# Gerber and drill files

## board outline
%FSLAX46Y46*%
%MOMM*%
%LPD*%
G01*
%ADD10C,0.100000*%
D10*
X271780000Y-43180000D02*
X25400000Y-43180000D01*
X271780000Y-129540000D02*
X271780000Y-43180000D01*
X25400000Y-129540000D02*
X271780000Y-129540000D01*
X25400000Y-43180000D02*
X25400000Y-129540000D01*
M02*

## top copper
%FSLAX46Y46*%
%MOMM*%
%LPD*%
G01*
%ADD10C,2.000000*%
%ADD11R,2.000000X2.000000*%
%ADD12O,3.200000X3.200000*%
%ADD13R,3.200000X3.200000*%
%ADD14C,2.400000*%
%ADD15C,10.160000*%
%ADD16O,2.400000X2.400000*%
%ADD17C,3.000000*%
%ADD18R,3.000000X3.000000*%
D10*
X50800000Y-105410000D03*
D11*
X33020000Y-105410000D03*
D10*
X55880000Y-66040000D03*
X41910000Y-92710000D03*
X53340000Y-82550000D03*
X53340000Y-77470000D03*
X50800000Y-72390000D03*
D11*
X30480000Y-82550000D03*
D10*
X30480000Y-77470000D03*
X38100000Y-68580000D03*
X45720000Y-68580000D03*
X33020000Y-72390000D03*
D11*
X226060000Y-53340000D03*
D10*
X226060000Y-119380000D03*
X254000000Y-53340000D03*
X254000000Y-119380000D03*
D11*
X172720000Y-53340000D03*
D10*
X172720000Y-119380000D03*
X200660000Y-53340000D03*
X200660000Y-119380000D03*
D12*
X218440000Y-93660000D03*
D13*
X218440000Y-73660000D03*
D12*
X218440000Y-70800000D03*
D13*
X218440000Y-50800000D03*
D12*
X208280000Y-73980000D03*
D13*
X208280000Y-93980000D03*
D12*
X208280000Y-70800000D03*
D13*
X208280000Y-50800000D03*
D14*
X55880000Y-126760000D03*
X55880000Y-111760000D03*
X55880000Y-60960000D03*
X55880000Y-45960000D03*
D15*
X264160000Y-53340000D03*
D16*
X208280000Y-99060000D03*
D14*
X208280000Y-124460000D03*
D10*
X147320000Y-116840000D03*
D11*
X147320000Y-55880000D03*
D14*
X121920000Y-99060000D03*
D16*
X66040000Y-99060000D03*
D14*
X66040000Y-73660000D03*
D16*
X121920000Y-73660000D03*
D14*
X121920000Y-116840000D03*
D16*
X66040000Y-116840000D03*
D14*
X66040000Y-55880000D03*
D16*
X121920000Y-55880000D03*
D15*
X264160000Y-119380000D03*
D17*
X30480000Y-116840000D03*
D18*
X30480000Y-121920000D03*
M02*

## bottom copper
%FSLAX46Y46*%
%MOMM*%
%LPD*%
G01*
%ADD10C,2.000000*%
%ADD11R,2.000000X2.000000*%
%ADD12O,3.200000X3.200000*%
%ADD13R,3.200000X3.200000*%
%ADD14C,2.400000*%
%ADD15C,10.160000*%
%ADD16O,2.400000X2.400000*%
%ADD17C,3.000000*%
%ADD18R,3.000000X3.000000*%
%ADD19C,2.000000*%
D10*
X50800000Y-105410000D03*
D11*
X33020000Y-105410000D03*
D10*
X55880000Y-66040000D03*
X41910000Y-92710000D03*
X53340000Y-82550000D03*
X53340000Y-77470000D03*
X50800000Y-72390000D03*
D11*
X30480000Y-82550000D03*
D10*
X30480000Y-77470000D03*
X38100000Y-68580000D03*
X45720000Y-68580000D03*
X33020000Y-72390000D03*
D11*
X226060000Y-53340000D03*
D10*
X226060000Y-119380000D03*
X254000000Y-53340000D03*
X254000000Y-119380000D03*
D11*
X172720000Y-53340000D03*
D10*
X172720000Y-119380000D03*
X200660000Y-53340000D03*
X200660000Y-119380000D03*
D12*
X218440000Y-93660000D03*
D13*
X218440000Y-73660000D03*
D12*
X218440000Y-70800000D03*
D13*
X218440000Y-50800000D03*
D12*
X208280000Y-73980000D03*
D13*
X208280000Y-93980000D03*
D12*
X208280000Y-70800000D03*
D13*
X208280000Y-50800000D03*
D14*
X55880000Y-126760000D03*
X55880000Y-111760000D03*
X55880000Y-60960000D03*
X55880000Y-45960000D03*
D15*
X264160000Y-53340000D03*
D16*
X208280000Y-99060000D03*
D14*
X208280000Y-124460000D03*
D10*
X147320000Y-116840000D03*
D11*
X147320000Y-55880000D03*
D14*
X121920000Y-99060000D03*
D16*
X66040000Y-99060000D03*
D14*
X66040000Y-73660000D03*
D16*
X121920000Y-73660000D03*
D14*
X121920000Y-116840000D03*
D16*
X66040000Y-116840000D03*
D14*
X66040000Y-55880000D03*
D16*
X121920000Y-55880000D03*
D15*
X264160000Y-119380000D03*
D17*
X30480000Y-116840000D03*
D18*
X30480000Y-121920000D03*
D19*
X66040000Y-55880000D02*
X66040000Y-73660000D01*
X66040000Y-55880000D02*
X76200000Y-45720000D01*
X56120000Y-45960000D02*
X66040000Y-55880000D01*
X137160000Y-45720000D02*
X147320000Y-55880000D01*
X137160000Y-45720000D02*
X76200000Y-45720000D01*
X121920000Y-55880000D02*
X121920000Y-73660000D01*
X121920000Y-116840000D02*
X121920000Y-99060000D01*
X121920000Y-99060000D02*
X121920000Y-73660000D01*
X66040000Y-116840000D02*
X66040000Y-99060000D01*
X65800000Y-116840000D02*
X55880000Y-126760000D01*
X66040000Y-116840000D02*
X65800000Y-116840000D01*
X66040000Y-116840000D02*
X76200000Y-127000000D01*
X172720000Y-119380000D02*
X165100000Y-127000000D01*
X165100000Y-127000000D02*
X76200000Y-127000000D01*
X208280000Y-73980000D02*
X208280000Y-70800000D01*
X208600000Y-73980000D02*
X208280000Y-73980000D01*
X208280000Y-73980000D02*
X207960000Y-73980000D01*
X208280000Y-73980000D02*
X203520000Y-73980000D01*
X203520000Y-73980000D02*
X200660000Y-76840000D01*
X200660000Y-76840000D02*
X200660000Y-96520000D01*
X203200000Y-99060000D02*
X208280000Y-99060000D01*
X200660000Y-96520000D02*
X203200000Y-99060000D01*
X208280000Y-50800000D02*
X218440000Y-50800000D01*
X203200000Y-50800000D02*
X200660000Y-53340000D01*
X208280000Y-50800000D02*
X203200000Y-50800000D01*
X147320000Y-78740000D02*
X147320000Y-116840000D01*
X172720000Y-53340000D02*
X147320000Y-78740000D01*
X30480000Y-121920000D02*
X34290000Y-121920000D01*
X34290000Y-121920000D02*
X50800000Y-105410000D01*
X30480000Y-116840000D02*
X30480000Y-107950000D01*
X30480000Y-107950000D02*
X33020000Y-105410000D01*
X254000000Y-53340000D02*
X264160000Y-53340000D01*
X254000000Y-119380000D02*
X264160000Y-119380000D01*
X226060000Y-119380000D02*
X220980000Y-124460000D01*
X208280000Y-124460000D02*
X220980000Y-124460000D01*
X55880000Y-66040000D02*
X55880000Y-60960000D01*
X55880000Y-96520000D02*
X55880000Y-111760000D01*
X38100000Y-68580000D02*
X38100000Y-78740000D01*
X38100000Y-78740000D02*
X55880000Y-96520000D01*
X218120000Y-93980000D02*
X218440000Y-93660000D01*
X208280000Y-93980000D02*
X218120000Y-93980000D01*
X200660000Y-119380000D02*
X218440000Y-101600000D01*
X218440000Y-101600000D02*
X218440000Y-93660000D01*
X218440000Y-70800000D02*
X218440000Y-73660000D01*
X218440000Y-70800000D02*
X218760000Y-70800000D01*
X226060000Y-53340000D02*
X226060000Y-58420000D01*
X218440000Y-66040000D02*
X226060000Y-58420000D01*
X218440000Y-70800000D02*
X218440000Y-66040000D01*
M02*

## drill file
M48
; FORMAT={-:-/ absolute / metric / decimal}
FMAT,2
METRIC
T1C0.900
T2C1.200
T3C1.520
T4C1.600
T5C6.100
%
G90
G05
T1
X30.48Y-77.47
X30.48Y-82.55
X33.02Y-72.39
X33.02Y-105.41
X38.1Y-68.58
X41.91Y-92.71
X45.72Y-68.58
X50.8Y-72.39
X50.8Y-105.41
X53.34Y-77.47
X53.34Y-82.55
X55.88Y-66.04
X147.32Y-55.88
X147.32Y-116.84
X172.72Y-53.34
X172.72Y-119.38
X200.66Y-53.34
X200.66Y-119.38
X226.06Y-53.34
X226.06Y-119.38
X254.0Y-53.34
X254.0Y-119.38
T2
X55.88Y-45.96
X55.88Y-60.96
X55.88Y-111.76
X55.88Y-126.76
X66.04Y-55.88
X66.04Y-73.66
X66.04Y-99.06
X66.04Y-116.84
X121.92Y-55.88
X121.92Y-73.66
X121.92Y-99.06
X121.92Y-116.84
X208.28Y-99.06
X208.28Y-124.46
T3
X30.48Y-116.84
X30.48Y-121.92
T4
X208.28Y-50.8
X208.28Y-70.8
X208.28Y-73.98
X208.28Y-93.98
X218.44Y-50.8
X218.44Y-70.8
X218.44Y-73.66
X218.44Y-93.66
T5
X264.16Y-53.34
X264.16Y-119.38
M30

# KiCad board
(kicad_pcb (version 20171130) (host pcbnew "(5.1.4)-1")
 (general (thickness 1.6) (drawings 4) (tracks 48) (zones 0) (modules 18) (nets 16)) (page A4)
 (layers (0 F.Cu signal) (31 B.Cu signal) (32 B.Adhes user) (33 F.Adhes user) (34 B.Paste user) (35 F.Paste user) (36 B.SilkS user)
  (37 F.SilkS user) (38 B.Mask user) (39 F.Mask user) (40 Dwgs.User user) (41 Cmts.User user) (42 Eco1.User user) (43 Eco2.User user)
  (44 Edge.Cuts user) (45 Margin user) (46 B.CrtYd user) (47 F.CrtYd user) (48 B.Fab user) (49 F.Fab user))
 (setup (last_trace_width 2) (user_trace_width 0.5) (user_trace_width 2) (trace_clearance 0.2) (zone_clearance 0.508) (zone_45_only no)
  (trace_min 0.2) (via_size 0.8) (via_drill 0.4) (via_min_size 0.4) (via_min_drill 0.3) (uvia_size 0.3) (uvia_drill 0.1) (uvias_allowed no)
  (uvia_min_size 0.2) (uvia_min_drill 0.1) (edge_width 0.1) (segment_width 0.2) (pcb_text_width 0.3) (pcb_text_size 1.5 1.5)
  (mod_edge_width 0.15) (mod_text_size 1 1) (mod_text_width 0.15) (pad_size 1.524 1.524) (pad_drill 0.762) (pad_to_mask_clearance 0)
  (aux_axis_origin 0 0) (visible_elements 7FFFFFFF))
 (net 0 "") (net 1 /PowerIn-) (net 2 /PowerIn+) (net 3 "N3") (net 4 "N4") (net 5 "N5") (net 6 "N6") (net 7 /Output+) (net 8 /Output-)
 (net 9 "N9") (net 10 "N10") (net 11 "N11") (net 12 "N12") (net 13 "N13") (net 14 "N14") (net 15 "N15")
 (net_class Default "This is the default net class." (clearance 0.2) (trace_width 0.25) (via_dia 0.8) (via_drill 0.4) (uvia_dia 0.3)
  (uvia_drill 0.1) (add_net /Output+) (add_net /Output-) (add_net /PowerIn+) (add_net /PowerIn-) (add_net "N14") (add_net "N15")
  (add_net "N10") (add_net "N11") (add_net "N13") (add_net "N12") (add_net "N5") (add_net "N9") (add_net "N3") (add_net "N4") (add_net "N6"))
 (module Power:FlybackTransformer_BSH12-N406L (layer F.Cu) (at 57.15 66.04 270)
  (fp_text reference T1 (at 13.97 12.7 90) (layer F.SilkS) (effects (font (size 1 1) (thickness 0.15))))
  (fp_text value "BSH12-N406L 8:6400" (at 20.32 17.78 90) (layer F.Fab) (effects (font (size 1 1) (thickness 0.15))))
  (pad 11 thru_hole circle (at 39.37 6.35 270) (size 2 2) (drill 0.9) (layers *.Cu *.Mask) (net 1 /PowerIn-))
  (pad 10 thru_hole rect (at 39.37 24.13 270) (size 2 2) (drill 0.9) (layers *.Cu *.Mask) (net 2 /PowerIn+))
  (pad 12 thru_hole circle (at 0 1.27 270) (size 2 2) (drill 0.9) (layers *.Cu *.Mask) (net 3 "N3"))
  (pad 9 thru_hole circle (at 26.67 15.24 270) (size 2 2) (drill 0.9) (layers *.Cu *.Mask))
  (pad 8 thru_hole circle (at 16.51 3.81 270) (size 2 2) (drill 0.9) (layers *.Cu *.Mask))
  (pad 7 thru_hole circle (at 11.43 3.81 270) (size 2 2) (drill 0.9) (layers *.Cu *.Mask))
  (pad 6 thru_hole circle (at 6.35 6.35 270) (size 2 2) (drill 0.9) (layers *.Cu *.Mask))
  (pad 1 thru_hole rect (at 16.51 26.67 270) (size 2 2) (drill 0.9) (layers *.Cu *.Mask))
  (pad 2 thru_hole circle (at 11.43 26.67 270) (size 2 2) (drill 0.9) (layers *.Cu *.Mask))
  (pad 4 thru_hole circle (at 2.54 19.05 270) (size 2 2) (drill 0.9) (layers *.Cu *.Mask) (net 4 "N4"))
  (pad 5 thru_hole circle (at 2.54 11.43 270) (size 2 2) (drill 0.9) (layers *.Cu *.Mask))
  (pad 3 thru_hole circle (at 6.35 24.13 270) (size 2 2) (drill 0.9) (layers *.Cu *.Mask)))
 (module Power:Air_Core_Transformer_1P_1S (layer F.Cu) (at 226.06 53.34)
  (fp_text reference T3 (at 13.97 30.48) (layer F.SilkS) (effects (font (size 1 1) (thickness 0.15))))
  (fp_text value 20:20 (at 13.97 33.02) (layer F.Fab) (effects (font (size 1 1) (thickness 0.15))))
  (pad 1 thru_hole rect (at 0 0) (size 2 2) (drill 0.9) (layers *.Cu *.Mask) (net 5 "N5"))
  (pad 2 thru_hole circle (at 0 66.04) (size 2 2) (drill 0.9) (layers *.Cu *.Mask) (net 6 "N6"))
  (pad 4 thru_hole circle (at 27.94 0) (size 2 2) (drill 0.9) (layers *.Cu *.Mask) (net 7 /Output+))
  (pad 3 thru_hole circle (at 27.94 66.04) (size 2 2) (drill 0.9) (layers *.Cu *.Mask) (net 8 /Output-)))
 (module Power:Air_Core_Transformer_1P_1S (layer F.Cu) (at 172.72 53.34)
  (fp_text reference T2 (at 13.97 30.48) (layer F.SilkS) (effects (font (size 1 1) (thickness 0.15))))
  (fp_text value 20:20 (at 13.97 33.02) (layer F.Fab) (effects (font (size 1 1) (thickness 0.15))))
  (pad 1 thru_hole rect (at 0 0) (size 2 2) (drill 0.9) (layers *.Cu *.Mask) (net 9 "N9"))
  (pad 2 thru_hole circle (at 0 66.04) (size 2 2) (drill 0.9) (layers *.Cu *.Mask) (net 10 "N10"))
  (pad 4 thru_hole circle (at 27.94 0) (size 2 2) (drill 0.9) (layers *.Cu *.Mask) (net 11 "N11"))
  (pad 3 thru_hole circle (at 27.94 66.04) (size 2 2) (drill 0.9) (layers *.Cu *.Mask) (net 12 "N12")))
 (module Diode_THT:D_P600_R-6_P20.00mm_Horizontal (layer F.Cu) (at 218.44 73.66 270)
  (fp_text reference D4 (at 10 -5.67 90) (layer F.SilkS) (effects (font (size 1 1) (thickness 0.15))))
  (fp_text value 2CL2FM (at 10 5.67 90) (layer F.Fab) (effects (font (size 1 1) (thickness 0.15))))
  (pad 2 thru_hole oval (at 20 0 270) (size 3.2 3.2) (drill 1.6) (layers *.Cu *.Mask) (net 12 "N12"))
  (pad 1 thru_hole rect (at 0 0 270) (size 3.2 3.2) (drill 1.6) (layers *.Cu *.Mask) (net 5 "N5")))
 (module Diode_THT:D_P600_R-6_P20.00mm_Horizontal (layer F.Cu) (at 218.44 50.8 270)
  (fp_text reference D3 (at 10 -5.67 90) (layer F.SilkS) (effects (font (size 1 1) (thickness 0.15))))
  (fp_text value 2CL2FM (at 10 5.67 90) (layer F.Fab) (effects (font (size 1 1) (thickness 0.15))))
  (pad 2 thru_hole oval (at 20 0 270) (size 3.2 3.2) (drill 1.6) (layers *.Cu *.Mask) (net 5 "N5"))
  (pad 1 thru_hole rect (at 0 0 270) (size 3.2 3.2) (drill 1.6) (layers *.Cu *.Mask) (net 11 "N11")))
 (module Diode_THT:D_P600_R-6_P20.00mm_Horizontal (layer F.Cu) (at 208.28 93.98 90)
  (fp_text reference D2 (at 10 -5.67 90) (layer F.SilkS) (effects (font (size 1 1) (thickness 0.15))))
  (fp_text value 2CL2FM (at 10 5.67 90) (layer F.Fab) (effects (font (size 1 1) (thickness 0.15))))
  (pad 2 thru_hole oval (at 20 0 90) (size 3.2 3.2) (drill 1.6) (layers *.Cu *.Mask) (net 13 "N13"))
  (pad 1 thru_hole rect (at 0 0 90) (size 3.2 3.2) (drill 1.6) (layers *.Cu *.Mask) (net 12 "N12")))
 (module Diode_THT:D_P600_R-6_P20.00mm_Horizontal (layer F.Cu) (at 208.28 50.8 270)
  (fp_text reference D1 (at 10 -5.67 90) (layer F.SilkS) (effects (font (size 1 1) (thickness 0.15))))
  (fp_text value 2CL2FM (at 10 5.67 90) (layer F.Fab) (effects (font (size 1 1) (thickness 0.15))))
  (pad 2 thru_hole oval (at 20 0 270) (size 3.2 3.2) (drill 1.6) (layers *.Cu *.Mask) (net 13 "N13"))
  (pad 1 thru_hole rect (at 0 0 270) (size 3.2 3.2) (drill 1.6) (layers *.Cu *.Mask) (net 11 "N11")))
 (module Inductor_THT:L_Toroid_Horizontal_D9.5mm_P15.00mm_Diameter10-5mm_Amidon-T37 (layer F.Cu) (at 55.88 111.76 270)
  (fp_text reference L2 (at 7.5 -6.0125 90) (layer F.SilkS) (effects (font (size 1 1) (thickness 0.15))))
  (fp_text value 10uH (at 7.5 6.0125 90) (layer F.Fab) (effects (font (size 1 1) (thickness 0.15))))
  (pad 2 thru_hole circle (at 15 0 270) (size 2.4 2.4) (drill 1.2) (layers *.Cu *.Mask) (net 10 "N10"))
  (pad 1 thru_hole circle (at 0 0 270) (size 2.4 2.4) (drill 1.2) (layers *.Cu *.Mask) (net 4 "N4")))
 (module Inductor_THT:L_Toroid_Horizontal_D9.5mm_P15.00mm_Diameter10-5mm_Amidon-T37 (layer F.Cu) (at 55.88 60.96 90)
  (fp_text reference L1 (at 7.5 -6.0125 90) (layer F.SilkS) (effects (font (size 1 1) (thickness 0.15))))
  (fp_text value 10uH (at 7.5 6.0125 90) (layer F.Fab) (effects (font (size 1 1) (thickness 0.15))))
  (pad 1 thru_hole circle (at 0 0 90) (size 2.4 2.4) (drill 1.2) (layers *.Cu *.Mask) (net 3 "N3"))
  (pad 2 thru_hole circle (at 15 0 90) (size 2.4 2.4) (drill 1.2) (layers *.Cu *.Mask) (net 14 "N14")))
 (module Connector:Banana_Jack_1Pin (layer F.Cu) (at 264.16 53.34)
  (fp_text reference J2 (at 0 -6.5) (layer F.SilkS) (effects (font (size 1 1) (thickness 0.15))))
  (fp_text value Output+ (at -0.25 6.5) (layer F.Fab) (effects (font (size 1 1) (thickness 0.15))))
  (pad 1 thru_hole circle (at 0 0) (size 10.16 10.16) (drill 6.1) (layers *.Cu *.Mask) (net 7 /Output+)))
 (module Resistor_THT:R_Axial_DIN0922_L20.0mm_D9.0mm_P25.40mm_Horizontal (layer F.Cu) (at 208.28 124.46 90)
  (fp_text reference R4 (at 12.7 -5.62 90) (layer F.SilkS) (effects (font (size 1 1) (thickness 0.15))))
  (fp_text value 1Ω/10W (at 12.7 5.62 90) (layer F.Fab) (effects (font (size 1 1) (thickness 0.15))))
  (pad 2 thru_hole oval (at 25.4 0 90) (size 2.4 2.4) (drill 1.2) (layers *.Cu *.Mask) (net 13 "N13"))
  (pad 1 thru_hole circle (at 0 0 90) (size 2.4 2.4) (drill 1.2) (layers *.Cu *.Mask) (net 6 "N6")))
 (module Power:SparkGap (layer F.Cu) (at 147.32 55.88 270)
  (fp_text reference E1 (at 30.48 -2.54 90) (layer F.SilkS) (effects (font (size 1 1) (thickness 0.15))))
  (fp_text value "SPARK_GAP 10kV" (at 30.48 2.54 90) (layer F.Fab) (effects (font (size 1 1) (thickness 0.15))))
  (pad 2 thru_hole circle (at 60.96 0 270) (size 2 2) (drill 0.9) (layers *.Cu *.Mask) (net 9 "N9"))
  (pad 1 thru_hole rect (at 0 0 270) (size 2 2) (drill 0.9) (layers *.Cu *.Mask) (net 14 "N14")))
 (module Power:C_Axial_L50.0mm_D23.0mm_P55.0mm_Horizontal (layer F.Cu) (at 121.92 99.06 180)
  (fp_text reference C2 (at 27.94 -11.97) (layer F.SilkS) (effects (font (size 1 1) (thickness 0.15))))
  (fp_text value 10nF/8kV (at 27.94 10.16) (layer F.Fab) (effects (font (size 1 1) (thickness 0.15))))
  (pad 1 thru_hole circle (at 0 0 180) (size 2.4 2.4) (drill 1.2) (layers *.Cu *.Mask) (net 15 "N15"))
  (pad 2 thru_hole oval (at 55.88 0 180) (size 2.4 2.4) (drill 1.2) (layers *.Cu *.Mask) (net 10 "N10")))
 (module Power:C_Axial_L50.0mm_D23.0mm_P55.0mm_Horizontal (layer F.Cu) (at 66.04 73.66)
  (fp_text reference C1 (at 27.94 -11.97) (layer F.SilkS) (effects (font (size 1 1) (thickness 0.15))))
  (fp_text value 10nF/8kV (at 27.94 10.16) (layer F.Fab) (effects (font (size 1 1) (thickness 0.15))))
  (pad 1 thru_hole circle (at 0 0) (size 2.4 2.4) (drill 1.2) (layers *.Cu *.Mask) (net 14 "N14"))
  (pad 2 thru_hole oval (at 55.88 0) (size 2.4 2.4) (drill 1.2) (layers *.Cu *.Mask) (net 15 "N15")))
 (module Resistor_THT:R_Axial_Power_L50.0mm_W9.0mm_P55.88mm (layer F.Cu) (at 121.92 116.84 180)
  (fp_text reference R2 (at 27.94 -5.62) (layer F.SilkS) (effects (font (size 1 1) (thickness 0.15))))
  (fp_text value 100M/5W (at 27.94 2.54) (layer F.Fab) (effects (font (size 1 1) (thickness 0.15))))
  (pad 1 thru_hole circle (at 0 0 180) (size 2.4 2.4) (drill 1.2) (layers *.Cu *.Mask) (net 15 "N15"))
  (pad 2 thru_hole oval (at 55.88 0 180) (size 2.4 2.4) (drill 1.2) (layers *.Cu *.Mask) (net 10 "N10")))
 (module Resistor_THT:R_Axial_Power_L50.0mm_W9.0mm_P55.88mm (layer F.Cu) (at 66.04 55.88)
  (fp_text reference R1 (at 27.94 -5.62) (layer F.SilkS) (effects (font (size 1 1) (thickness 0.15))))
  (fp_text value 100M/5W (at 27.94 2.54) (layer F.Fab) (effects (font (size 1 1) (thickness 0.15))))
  (pad 1 thru_hole circle (at 0 0) (size 2.4 2.4) (drill 1.2) (layers *.Cu *.Mask) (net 14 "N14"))
  (pad 2 thru_hole oval (at 55.88 0) (size 2.4 2.4) (drill 1.2) (layers *.Cu *.Mask) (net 15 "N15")))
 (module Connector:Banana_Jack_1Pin (layer F.Cu) (at 264.16 119.38)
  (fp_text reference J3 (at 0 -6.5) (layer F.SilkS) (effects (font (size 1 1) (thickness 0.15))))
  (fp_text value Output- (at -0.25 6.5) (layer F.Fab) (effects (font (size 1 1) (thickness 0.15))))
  (pad 1 thru_hole circle (at 0 0) (size 10.16 10.16) (drill 6.1) (layers *.Cu *.Mask) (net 8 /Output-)))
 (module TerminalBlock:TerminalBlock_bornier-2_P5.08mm (layer F.Cu) (at 30.48 121.92 90)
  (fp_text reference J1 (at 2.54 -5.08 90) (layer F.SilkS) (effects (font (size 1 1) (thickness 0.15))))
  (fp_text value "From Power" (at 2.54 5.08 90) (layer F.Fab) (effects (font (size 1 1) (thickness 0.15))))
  (pad 2 thru_hole circle (at 5.08 0 90) (size 3 3) (drill 1.52) (layers *.Cu *.Mask) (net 2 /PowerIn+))
  (pad 1 thru_hole rect (at 0 0 90) (size 3 3) (drill 1.52) (layers *.Cu *.Mask) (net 1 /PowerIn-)))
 (gr_line (start 271.78 43.18) (end 25.4 43.18) (layer Edge.Cuts) (width 0.1))
 (gr_line (start 271.78 129.54) (end 271.78 43.18) (layer Edge.Cuts) (width 0.1))
 (gr_line (start 25.4 129.54) (end 271.78 129.54) (layer Edge.Cuts) (width 0.1))
 (gr_line (start 25.4 43.18) (end 25.4 129.54) (layer Edge.Cuts) (width 0.1))
 (segment (start 66.04 55.88) (end 66.04 73.66) (width 2) (layer B.Cu) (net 14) (status 30))
 (segment (start 66.04 55.88) (end 76.2 45.72) (width 2) (layer B.Cu) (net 14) (status 10))
 (segment (start 56.12 45.96) (end 66.04 55.88) (width 2) (layer B.Cu) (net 14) (status 30))
 (segment (start 137.16 45.72) (end 147.32 55.88) (width 2) (layer B.Cu) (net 14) (status 20))
 (segment (start 137.16 45.72) (end 76.2 45.72) (width 2) (layer B.Cu) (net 14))
 (segment (start 121.92 55.88) (end 121.92 73.66) (width 2) (layer B.Cu) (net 15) (status 30))
 (segment (start 121.92 116.84) (end 121.92 99.06) (width 2) (layer B.Cu) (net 15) (status 30))
 (segment (start 121.92 99.06) (end 121.92 73.66) (width 2) (layer B.Cu) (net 15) (status 30))
 (segment (start 66.04 116.84) (end 66.04 99.06) (width 2) (layer B.Cu) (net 10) (status 30))
 (segment (start 65.8 116.84) (end 55.88 126.76) (width 2) (layer B.Cu) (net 10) (status 30))
 (segment (start 66.04 116.84) (end 65.8 116.84) (width 2) (layer B.Cu) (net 10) (status 30))
 (segment (start 66.04 116.84) (end 76.2 127) (width 2) (layer B.Cu) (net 10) (status 10))
 (segment (start 172.72 119.38) (end 165.1 127) (width 2) (layer B.Cu) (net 10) (status 10))
 (segment (start 165.1 127) (end 76.2 127) (width 2) (layer B.Cu) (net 10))
 (segment (start 208.28 73.98) (end 208.28 70.8) (width 2) (layer B.Cu) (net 13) (status 30))
 (segment (start 208.6 73.98) (end 208.28 73.98) (width 2) (layer B.Cu) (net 13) (status 30))
 (segment (start 208.28 73.98) (end 207.96 73.98) (width 2) (layer B.Cu) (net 13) (status 30))
 (segment (start 208.28 73.98) (end 203.52 73.98) (width 2) (layer B.Cu) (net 13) (status 10))
 (segment (start 203.52 73.98) (end 200.66 76.84) (width 2) (layer B.Cu) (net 13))
 (segment (start 200.66 76.84) (end 200.66 96.52) (width 2) (layer B.Cu) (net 13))
 (segment (start 203.2 99.06) (end 208.28 99.06) (width 2) (layer B.Cu) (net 13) (status 20))
 (segment (start 200.66 96.52) (end 203.2 99.06) (width 2) (layer B.Cu) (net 13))
 (segment (start 208.28 50.8) (end 218.44 50.8) (width 2) (layer B.Cu) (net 11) (status 30))
 (segment (start 203.2 50.8) (end 200.66 53.34) (width 2) (layer B.Cu) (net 11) (status 20))
 (segment (start 208.28 50.8) (end 203.2 50.8) (width 2) (layer B.Cu) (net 11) (status 10))
 (segment (start 147.32 78.74) (end 147.32 116.84) (width 2) (layer B.Cu) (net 9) (status 20))
 (segment (start 172.72 53.34) (end 147.32 78.74) (width 2) (layer B.Cu) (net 9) (status 10))
 (segment (start 30.48 121.92) (end 34.29 121.92) (width 2) (layer B.Cu) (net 1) (status 10))
 (segment (start 34.29 121.92) (end 50.8 105.41) (width 2) (layer B.Cu) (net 1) (status 20))
 (segment (start 30.48 116.84) (end 30.48 107.95) (width 2) (layer B.Cu) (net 2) (status 10))
 (segment (start 30.48 107.95) (end 33.02 105.41) (width 2) (layer B.Cu) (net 2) (status 20))
 (segment (start 254 53.34) (end 264.16 53.34) (width 2) (layer B.Cu) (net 7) (status 30))
 (segment (start 254 119.38) (end 264.16 119.38) (width 2) (layer B.Cu) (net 8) (status 30))
 (segment (start 226.06 119.38) (end 220.98 124.46) (width 2) (layer B.Cu) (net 6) (status 10))
 (segment (start 208.28 124.46) (end 220.98 124.46) (width 2) (layer B.Cu) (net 6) (status 10))
 (segment (start 55.88 66.04) (end 55.88 60.96) (width 2) (layer B.Cu) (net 3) (status 30))
 (segment (start 55.88 96.52) (end 55.88 111.76) (width 2) (layer B.Cu) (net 4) (status 20))
 (segment (start 38.1 68.58) (end 38.1 78.74) (width 2) (layer B.Cu) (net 4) (status 10))
 (segment (start 38.1 78.74) (end 55.88 96.52) (width 2) (layer B.Cu) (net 4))
 (segment (start 218.12 93.98) (end 218.44 93.66) (width 2) (layer B.Cu) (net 12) (status 30))
 (segment (start 208.28 93.98) (end 218.12 93.98) (width 2) (layer B.Cu) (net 12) (status 30))
 (segment (start 200.66 119.38) (end 218.44 101.6) (width 2) (layer B.Cu) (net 12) (status 10))
 (segment (start 218.44 101.6) (end 218.44 93.66) (width 2) (layer B.Cu) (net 12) (status 20))
 (segment (start 218.44 70.8) (end 218.44 73.66) (width 2) (layer B.Cu) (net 5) (status 30))
 (segment (start 218.44 70.8) (end 218.76 70.8) (width 2) (layer B.Cu) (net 5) (status 30))
 (segment (start 226.06 53.34) (end 226.06 58.42) (width 2) (layer B.Cu) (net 5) (status 10))
 (segment (start 218.44 66.04) (end 226.06 58.42) (width 2) (layer B.Cu) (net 5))
 (segment (start 218.44 70.8) (end 218.44 66.04) (width 2) (layer B.Cu) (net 5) (status 10)))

